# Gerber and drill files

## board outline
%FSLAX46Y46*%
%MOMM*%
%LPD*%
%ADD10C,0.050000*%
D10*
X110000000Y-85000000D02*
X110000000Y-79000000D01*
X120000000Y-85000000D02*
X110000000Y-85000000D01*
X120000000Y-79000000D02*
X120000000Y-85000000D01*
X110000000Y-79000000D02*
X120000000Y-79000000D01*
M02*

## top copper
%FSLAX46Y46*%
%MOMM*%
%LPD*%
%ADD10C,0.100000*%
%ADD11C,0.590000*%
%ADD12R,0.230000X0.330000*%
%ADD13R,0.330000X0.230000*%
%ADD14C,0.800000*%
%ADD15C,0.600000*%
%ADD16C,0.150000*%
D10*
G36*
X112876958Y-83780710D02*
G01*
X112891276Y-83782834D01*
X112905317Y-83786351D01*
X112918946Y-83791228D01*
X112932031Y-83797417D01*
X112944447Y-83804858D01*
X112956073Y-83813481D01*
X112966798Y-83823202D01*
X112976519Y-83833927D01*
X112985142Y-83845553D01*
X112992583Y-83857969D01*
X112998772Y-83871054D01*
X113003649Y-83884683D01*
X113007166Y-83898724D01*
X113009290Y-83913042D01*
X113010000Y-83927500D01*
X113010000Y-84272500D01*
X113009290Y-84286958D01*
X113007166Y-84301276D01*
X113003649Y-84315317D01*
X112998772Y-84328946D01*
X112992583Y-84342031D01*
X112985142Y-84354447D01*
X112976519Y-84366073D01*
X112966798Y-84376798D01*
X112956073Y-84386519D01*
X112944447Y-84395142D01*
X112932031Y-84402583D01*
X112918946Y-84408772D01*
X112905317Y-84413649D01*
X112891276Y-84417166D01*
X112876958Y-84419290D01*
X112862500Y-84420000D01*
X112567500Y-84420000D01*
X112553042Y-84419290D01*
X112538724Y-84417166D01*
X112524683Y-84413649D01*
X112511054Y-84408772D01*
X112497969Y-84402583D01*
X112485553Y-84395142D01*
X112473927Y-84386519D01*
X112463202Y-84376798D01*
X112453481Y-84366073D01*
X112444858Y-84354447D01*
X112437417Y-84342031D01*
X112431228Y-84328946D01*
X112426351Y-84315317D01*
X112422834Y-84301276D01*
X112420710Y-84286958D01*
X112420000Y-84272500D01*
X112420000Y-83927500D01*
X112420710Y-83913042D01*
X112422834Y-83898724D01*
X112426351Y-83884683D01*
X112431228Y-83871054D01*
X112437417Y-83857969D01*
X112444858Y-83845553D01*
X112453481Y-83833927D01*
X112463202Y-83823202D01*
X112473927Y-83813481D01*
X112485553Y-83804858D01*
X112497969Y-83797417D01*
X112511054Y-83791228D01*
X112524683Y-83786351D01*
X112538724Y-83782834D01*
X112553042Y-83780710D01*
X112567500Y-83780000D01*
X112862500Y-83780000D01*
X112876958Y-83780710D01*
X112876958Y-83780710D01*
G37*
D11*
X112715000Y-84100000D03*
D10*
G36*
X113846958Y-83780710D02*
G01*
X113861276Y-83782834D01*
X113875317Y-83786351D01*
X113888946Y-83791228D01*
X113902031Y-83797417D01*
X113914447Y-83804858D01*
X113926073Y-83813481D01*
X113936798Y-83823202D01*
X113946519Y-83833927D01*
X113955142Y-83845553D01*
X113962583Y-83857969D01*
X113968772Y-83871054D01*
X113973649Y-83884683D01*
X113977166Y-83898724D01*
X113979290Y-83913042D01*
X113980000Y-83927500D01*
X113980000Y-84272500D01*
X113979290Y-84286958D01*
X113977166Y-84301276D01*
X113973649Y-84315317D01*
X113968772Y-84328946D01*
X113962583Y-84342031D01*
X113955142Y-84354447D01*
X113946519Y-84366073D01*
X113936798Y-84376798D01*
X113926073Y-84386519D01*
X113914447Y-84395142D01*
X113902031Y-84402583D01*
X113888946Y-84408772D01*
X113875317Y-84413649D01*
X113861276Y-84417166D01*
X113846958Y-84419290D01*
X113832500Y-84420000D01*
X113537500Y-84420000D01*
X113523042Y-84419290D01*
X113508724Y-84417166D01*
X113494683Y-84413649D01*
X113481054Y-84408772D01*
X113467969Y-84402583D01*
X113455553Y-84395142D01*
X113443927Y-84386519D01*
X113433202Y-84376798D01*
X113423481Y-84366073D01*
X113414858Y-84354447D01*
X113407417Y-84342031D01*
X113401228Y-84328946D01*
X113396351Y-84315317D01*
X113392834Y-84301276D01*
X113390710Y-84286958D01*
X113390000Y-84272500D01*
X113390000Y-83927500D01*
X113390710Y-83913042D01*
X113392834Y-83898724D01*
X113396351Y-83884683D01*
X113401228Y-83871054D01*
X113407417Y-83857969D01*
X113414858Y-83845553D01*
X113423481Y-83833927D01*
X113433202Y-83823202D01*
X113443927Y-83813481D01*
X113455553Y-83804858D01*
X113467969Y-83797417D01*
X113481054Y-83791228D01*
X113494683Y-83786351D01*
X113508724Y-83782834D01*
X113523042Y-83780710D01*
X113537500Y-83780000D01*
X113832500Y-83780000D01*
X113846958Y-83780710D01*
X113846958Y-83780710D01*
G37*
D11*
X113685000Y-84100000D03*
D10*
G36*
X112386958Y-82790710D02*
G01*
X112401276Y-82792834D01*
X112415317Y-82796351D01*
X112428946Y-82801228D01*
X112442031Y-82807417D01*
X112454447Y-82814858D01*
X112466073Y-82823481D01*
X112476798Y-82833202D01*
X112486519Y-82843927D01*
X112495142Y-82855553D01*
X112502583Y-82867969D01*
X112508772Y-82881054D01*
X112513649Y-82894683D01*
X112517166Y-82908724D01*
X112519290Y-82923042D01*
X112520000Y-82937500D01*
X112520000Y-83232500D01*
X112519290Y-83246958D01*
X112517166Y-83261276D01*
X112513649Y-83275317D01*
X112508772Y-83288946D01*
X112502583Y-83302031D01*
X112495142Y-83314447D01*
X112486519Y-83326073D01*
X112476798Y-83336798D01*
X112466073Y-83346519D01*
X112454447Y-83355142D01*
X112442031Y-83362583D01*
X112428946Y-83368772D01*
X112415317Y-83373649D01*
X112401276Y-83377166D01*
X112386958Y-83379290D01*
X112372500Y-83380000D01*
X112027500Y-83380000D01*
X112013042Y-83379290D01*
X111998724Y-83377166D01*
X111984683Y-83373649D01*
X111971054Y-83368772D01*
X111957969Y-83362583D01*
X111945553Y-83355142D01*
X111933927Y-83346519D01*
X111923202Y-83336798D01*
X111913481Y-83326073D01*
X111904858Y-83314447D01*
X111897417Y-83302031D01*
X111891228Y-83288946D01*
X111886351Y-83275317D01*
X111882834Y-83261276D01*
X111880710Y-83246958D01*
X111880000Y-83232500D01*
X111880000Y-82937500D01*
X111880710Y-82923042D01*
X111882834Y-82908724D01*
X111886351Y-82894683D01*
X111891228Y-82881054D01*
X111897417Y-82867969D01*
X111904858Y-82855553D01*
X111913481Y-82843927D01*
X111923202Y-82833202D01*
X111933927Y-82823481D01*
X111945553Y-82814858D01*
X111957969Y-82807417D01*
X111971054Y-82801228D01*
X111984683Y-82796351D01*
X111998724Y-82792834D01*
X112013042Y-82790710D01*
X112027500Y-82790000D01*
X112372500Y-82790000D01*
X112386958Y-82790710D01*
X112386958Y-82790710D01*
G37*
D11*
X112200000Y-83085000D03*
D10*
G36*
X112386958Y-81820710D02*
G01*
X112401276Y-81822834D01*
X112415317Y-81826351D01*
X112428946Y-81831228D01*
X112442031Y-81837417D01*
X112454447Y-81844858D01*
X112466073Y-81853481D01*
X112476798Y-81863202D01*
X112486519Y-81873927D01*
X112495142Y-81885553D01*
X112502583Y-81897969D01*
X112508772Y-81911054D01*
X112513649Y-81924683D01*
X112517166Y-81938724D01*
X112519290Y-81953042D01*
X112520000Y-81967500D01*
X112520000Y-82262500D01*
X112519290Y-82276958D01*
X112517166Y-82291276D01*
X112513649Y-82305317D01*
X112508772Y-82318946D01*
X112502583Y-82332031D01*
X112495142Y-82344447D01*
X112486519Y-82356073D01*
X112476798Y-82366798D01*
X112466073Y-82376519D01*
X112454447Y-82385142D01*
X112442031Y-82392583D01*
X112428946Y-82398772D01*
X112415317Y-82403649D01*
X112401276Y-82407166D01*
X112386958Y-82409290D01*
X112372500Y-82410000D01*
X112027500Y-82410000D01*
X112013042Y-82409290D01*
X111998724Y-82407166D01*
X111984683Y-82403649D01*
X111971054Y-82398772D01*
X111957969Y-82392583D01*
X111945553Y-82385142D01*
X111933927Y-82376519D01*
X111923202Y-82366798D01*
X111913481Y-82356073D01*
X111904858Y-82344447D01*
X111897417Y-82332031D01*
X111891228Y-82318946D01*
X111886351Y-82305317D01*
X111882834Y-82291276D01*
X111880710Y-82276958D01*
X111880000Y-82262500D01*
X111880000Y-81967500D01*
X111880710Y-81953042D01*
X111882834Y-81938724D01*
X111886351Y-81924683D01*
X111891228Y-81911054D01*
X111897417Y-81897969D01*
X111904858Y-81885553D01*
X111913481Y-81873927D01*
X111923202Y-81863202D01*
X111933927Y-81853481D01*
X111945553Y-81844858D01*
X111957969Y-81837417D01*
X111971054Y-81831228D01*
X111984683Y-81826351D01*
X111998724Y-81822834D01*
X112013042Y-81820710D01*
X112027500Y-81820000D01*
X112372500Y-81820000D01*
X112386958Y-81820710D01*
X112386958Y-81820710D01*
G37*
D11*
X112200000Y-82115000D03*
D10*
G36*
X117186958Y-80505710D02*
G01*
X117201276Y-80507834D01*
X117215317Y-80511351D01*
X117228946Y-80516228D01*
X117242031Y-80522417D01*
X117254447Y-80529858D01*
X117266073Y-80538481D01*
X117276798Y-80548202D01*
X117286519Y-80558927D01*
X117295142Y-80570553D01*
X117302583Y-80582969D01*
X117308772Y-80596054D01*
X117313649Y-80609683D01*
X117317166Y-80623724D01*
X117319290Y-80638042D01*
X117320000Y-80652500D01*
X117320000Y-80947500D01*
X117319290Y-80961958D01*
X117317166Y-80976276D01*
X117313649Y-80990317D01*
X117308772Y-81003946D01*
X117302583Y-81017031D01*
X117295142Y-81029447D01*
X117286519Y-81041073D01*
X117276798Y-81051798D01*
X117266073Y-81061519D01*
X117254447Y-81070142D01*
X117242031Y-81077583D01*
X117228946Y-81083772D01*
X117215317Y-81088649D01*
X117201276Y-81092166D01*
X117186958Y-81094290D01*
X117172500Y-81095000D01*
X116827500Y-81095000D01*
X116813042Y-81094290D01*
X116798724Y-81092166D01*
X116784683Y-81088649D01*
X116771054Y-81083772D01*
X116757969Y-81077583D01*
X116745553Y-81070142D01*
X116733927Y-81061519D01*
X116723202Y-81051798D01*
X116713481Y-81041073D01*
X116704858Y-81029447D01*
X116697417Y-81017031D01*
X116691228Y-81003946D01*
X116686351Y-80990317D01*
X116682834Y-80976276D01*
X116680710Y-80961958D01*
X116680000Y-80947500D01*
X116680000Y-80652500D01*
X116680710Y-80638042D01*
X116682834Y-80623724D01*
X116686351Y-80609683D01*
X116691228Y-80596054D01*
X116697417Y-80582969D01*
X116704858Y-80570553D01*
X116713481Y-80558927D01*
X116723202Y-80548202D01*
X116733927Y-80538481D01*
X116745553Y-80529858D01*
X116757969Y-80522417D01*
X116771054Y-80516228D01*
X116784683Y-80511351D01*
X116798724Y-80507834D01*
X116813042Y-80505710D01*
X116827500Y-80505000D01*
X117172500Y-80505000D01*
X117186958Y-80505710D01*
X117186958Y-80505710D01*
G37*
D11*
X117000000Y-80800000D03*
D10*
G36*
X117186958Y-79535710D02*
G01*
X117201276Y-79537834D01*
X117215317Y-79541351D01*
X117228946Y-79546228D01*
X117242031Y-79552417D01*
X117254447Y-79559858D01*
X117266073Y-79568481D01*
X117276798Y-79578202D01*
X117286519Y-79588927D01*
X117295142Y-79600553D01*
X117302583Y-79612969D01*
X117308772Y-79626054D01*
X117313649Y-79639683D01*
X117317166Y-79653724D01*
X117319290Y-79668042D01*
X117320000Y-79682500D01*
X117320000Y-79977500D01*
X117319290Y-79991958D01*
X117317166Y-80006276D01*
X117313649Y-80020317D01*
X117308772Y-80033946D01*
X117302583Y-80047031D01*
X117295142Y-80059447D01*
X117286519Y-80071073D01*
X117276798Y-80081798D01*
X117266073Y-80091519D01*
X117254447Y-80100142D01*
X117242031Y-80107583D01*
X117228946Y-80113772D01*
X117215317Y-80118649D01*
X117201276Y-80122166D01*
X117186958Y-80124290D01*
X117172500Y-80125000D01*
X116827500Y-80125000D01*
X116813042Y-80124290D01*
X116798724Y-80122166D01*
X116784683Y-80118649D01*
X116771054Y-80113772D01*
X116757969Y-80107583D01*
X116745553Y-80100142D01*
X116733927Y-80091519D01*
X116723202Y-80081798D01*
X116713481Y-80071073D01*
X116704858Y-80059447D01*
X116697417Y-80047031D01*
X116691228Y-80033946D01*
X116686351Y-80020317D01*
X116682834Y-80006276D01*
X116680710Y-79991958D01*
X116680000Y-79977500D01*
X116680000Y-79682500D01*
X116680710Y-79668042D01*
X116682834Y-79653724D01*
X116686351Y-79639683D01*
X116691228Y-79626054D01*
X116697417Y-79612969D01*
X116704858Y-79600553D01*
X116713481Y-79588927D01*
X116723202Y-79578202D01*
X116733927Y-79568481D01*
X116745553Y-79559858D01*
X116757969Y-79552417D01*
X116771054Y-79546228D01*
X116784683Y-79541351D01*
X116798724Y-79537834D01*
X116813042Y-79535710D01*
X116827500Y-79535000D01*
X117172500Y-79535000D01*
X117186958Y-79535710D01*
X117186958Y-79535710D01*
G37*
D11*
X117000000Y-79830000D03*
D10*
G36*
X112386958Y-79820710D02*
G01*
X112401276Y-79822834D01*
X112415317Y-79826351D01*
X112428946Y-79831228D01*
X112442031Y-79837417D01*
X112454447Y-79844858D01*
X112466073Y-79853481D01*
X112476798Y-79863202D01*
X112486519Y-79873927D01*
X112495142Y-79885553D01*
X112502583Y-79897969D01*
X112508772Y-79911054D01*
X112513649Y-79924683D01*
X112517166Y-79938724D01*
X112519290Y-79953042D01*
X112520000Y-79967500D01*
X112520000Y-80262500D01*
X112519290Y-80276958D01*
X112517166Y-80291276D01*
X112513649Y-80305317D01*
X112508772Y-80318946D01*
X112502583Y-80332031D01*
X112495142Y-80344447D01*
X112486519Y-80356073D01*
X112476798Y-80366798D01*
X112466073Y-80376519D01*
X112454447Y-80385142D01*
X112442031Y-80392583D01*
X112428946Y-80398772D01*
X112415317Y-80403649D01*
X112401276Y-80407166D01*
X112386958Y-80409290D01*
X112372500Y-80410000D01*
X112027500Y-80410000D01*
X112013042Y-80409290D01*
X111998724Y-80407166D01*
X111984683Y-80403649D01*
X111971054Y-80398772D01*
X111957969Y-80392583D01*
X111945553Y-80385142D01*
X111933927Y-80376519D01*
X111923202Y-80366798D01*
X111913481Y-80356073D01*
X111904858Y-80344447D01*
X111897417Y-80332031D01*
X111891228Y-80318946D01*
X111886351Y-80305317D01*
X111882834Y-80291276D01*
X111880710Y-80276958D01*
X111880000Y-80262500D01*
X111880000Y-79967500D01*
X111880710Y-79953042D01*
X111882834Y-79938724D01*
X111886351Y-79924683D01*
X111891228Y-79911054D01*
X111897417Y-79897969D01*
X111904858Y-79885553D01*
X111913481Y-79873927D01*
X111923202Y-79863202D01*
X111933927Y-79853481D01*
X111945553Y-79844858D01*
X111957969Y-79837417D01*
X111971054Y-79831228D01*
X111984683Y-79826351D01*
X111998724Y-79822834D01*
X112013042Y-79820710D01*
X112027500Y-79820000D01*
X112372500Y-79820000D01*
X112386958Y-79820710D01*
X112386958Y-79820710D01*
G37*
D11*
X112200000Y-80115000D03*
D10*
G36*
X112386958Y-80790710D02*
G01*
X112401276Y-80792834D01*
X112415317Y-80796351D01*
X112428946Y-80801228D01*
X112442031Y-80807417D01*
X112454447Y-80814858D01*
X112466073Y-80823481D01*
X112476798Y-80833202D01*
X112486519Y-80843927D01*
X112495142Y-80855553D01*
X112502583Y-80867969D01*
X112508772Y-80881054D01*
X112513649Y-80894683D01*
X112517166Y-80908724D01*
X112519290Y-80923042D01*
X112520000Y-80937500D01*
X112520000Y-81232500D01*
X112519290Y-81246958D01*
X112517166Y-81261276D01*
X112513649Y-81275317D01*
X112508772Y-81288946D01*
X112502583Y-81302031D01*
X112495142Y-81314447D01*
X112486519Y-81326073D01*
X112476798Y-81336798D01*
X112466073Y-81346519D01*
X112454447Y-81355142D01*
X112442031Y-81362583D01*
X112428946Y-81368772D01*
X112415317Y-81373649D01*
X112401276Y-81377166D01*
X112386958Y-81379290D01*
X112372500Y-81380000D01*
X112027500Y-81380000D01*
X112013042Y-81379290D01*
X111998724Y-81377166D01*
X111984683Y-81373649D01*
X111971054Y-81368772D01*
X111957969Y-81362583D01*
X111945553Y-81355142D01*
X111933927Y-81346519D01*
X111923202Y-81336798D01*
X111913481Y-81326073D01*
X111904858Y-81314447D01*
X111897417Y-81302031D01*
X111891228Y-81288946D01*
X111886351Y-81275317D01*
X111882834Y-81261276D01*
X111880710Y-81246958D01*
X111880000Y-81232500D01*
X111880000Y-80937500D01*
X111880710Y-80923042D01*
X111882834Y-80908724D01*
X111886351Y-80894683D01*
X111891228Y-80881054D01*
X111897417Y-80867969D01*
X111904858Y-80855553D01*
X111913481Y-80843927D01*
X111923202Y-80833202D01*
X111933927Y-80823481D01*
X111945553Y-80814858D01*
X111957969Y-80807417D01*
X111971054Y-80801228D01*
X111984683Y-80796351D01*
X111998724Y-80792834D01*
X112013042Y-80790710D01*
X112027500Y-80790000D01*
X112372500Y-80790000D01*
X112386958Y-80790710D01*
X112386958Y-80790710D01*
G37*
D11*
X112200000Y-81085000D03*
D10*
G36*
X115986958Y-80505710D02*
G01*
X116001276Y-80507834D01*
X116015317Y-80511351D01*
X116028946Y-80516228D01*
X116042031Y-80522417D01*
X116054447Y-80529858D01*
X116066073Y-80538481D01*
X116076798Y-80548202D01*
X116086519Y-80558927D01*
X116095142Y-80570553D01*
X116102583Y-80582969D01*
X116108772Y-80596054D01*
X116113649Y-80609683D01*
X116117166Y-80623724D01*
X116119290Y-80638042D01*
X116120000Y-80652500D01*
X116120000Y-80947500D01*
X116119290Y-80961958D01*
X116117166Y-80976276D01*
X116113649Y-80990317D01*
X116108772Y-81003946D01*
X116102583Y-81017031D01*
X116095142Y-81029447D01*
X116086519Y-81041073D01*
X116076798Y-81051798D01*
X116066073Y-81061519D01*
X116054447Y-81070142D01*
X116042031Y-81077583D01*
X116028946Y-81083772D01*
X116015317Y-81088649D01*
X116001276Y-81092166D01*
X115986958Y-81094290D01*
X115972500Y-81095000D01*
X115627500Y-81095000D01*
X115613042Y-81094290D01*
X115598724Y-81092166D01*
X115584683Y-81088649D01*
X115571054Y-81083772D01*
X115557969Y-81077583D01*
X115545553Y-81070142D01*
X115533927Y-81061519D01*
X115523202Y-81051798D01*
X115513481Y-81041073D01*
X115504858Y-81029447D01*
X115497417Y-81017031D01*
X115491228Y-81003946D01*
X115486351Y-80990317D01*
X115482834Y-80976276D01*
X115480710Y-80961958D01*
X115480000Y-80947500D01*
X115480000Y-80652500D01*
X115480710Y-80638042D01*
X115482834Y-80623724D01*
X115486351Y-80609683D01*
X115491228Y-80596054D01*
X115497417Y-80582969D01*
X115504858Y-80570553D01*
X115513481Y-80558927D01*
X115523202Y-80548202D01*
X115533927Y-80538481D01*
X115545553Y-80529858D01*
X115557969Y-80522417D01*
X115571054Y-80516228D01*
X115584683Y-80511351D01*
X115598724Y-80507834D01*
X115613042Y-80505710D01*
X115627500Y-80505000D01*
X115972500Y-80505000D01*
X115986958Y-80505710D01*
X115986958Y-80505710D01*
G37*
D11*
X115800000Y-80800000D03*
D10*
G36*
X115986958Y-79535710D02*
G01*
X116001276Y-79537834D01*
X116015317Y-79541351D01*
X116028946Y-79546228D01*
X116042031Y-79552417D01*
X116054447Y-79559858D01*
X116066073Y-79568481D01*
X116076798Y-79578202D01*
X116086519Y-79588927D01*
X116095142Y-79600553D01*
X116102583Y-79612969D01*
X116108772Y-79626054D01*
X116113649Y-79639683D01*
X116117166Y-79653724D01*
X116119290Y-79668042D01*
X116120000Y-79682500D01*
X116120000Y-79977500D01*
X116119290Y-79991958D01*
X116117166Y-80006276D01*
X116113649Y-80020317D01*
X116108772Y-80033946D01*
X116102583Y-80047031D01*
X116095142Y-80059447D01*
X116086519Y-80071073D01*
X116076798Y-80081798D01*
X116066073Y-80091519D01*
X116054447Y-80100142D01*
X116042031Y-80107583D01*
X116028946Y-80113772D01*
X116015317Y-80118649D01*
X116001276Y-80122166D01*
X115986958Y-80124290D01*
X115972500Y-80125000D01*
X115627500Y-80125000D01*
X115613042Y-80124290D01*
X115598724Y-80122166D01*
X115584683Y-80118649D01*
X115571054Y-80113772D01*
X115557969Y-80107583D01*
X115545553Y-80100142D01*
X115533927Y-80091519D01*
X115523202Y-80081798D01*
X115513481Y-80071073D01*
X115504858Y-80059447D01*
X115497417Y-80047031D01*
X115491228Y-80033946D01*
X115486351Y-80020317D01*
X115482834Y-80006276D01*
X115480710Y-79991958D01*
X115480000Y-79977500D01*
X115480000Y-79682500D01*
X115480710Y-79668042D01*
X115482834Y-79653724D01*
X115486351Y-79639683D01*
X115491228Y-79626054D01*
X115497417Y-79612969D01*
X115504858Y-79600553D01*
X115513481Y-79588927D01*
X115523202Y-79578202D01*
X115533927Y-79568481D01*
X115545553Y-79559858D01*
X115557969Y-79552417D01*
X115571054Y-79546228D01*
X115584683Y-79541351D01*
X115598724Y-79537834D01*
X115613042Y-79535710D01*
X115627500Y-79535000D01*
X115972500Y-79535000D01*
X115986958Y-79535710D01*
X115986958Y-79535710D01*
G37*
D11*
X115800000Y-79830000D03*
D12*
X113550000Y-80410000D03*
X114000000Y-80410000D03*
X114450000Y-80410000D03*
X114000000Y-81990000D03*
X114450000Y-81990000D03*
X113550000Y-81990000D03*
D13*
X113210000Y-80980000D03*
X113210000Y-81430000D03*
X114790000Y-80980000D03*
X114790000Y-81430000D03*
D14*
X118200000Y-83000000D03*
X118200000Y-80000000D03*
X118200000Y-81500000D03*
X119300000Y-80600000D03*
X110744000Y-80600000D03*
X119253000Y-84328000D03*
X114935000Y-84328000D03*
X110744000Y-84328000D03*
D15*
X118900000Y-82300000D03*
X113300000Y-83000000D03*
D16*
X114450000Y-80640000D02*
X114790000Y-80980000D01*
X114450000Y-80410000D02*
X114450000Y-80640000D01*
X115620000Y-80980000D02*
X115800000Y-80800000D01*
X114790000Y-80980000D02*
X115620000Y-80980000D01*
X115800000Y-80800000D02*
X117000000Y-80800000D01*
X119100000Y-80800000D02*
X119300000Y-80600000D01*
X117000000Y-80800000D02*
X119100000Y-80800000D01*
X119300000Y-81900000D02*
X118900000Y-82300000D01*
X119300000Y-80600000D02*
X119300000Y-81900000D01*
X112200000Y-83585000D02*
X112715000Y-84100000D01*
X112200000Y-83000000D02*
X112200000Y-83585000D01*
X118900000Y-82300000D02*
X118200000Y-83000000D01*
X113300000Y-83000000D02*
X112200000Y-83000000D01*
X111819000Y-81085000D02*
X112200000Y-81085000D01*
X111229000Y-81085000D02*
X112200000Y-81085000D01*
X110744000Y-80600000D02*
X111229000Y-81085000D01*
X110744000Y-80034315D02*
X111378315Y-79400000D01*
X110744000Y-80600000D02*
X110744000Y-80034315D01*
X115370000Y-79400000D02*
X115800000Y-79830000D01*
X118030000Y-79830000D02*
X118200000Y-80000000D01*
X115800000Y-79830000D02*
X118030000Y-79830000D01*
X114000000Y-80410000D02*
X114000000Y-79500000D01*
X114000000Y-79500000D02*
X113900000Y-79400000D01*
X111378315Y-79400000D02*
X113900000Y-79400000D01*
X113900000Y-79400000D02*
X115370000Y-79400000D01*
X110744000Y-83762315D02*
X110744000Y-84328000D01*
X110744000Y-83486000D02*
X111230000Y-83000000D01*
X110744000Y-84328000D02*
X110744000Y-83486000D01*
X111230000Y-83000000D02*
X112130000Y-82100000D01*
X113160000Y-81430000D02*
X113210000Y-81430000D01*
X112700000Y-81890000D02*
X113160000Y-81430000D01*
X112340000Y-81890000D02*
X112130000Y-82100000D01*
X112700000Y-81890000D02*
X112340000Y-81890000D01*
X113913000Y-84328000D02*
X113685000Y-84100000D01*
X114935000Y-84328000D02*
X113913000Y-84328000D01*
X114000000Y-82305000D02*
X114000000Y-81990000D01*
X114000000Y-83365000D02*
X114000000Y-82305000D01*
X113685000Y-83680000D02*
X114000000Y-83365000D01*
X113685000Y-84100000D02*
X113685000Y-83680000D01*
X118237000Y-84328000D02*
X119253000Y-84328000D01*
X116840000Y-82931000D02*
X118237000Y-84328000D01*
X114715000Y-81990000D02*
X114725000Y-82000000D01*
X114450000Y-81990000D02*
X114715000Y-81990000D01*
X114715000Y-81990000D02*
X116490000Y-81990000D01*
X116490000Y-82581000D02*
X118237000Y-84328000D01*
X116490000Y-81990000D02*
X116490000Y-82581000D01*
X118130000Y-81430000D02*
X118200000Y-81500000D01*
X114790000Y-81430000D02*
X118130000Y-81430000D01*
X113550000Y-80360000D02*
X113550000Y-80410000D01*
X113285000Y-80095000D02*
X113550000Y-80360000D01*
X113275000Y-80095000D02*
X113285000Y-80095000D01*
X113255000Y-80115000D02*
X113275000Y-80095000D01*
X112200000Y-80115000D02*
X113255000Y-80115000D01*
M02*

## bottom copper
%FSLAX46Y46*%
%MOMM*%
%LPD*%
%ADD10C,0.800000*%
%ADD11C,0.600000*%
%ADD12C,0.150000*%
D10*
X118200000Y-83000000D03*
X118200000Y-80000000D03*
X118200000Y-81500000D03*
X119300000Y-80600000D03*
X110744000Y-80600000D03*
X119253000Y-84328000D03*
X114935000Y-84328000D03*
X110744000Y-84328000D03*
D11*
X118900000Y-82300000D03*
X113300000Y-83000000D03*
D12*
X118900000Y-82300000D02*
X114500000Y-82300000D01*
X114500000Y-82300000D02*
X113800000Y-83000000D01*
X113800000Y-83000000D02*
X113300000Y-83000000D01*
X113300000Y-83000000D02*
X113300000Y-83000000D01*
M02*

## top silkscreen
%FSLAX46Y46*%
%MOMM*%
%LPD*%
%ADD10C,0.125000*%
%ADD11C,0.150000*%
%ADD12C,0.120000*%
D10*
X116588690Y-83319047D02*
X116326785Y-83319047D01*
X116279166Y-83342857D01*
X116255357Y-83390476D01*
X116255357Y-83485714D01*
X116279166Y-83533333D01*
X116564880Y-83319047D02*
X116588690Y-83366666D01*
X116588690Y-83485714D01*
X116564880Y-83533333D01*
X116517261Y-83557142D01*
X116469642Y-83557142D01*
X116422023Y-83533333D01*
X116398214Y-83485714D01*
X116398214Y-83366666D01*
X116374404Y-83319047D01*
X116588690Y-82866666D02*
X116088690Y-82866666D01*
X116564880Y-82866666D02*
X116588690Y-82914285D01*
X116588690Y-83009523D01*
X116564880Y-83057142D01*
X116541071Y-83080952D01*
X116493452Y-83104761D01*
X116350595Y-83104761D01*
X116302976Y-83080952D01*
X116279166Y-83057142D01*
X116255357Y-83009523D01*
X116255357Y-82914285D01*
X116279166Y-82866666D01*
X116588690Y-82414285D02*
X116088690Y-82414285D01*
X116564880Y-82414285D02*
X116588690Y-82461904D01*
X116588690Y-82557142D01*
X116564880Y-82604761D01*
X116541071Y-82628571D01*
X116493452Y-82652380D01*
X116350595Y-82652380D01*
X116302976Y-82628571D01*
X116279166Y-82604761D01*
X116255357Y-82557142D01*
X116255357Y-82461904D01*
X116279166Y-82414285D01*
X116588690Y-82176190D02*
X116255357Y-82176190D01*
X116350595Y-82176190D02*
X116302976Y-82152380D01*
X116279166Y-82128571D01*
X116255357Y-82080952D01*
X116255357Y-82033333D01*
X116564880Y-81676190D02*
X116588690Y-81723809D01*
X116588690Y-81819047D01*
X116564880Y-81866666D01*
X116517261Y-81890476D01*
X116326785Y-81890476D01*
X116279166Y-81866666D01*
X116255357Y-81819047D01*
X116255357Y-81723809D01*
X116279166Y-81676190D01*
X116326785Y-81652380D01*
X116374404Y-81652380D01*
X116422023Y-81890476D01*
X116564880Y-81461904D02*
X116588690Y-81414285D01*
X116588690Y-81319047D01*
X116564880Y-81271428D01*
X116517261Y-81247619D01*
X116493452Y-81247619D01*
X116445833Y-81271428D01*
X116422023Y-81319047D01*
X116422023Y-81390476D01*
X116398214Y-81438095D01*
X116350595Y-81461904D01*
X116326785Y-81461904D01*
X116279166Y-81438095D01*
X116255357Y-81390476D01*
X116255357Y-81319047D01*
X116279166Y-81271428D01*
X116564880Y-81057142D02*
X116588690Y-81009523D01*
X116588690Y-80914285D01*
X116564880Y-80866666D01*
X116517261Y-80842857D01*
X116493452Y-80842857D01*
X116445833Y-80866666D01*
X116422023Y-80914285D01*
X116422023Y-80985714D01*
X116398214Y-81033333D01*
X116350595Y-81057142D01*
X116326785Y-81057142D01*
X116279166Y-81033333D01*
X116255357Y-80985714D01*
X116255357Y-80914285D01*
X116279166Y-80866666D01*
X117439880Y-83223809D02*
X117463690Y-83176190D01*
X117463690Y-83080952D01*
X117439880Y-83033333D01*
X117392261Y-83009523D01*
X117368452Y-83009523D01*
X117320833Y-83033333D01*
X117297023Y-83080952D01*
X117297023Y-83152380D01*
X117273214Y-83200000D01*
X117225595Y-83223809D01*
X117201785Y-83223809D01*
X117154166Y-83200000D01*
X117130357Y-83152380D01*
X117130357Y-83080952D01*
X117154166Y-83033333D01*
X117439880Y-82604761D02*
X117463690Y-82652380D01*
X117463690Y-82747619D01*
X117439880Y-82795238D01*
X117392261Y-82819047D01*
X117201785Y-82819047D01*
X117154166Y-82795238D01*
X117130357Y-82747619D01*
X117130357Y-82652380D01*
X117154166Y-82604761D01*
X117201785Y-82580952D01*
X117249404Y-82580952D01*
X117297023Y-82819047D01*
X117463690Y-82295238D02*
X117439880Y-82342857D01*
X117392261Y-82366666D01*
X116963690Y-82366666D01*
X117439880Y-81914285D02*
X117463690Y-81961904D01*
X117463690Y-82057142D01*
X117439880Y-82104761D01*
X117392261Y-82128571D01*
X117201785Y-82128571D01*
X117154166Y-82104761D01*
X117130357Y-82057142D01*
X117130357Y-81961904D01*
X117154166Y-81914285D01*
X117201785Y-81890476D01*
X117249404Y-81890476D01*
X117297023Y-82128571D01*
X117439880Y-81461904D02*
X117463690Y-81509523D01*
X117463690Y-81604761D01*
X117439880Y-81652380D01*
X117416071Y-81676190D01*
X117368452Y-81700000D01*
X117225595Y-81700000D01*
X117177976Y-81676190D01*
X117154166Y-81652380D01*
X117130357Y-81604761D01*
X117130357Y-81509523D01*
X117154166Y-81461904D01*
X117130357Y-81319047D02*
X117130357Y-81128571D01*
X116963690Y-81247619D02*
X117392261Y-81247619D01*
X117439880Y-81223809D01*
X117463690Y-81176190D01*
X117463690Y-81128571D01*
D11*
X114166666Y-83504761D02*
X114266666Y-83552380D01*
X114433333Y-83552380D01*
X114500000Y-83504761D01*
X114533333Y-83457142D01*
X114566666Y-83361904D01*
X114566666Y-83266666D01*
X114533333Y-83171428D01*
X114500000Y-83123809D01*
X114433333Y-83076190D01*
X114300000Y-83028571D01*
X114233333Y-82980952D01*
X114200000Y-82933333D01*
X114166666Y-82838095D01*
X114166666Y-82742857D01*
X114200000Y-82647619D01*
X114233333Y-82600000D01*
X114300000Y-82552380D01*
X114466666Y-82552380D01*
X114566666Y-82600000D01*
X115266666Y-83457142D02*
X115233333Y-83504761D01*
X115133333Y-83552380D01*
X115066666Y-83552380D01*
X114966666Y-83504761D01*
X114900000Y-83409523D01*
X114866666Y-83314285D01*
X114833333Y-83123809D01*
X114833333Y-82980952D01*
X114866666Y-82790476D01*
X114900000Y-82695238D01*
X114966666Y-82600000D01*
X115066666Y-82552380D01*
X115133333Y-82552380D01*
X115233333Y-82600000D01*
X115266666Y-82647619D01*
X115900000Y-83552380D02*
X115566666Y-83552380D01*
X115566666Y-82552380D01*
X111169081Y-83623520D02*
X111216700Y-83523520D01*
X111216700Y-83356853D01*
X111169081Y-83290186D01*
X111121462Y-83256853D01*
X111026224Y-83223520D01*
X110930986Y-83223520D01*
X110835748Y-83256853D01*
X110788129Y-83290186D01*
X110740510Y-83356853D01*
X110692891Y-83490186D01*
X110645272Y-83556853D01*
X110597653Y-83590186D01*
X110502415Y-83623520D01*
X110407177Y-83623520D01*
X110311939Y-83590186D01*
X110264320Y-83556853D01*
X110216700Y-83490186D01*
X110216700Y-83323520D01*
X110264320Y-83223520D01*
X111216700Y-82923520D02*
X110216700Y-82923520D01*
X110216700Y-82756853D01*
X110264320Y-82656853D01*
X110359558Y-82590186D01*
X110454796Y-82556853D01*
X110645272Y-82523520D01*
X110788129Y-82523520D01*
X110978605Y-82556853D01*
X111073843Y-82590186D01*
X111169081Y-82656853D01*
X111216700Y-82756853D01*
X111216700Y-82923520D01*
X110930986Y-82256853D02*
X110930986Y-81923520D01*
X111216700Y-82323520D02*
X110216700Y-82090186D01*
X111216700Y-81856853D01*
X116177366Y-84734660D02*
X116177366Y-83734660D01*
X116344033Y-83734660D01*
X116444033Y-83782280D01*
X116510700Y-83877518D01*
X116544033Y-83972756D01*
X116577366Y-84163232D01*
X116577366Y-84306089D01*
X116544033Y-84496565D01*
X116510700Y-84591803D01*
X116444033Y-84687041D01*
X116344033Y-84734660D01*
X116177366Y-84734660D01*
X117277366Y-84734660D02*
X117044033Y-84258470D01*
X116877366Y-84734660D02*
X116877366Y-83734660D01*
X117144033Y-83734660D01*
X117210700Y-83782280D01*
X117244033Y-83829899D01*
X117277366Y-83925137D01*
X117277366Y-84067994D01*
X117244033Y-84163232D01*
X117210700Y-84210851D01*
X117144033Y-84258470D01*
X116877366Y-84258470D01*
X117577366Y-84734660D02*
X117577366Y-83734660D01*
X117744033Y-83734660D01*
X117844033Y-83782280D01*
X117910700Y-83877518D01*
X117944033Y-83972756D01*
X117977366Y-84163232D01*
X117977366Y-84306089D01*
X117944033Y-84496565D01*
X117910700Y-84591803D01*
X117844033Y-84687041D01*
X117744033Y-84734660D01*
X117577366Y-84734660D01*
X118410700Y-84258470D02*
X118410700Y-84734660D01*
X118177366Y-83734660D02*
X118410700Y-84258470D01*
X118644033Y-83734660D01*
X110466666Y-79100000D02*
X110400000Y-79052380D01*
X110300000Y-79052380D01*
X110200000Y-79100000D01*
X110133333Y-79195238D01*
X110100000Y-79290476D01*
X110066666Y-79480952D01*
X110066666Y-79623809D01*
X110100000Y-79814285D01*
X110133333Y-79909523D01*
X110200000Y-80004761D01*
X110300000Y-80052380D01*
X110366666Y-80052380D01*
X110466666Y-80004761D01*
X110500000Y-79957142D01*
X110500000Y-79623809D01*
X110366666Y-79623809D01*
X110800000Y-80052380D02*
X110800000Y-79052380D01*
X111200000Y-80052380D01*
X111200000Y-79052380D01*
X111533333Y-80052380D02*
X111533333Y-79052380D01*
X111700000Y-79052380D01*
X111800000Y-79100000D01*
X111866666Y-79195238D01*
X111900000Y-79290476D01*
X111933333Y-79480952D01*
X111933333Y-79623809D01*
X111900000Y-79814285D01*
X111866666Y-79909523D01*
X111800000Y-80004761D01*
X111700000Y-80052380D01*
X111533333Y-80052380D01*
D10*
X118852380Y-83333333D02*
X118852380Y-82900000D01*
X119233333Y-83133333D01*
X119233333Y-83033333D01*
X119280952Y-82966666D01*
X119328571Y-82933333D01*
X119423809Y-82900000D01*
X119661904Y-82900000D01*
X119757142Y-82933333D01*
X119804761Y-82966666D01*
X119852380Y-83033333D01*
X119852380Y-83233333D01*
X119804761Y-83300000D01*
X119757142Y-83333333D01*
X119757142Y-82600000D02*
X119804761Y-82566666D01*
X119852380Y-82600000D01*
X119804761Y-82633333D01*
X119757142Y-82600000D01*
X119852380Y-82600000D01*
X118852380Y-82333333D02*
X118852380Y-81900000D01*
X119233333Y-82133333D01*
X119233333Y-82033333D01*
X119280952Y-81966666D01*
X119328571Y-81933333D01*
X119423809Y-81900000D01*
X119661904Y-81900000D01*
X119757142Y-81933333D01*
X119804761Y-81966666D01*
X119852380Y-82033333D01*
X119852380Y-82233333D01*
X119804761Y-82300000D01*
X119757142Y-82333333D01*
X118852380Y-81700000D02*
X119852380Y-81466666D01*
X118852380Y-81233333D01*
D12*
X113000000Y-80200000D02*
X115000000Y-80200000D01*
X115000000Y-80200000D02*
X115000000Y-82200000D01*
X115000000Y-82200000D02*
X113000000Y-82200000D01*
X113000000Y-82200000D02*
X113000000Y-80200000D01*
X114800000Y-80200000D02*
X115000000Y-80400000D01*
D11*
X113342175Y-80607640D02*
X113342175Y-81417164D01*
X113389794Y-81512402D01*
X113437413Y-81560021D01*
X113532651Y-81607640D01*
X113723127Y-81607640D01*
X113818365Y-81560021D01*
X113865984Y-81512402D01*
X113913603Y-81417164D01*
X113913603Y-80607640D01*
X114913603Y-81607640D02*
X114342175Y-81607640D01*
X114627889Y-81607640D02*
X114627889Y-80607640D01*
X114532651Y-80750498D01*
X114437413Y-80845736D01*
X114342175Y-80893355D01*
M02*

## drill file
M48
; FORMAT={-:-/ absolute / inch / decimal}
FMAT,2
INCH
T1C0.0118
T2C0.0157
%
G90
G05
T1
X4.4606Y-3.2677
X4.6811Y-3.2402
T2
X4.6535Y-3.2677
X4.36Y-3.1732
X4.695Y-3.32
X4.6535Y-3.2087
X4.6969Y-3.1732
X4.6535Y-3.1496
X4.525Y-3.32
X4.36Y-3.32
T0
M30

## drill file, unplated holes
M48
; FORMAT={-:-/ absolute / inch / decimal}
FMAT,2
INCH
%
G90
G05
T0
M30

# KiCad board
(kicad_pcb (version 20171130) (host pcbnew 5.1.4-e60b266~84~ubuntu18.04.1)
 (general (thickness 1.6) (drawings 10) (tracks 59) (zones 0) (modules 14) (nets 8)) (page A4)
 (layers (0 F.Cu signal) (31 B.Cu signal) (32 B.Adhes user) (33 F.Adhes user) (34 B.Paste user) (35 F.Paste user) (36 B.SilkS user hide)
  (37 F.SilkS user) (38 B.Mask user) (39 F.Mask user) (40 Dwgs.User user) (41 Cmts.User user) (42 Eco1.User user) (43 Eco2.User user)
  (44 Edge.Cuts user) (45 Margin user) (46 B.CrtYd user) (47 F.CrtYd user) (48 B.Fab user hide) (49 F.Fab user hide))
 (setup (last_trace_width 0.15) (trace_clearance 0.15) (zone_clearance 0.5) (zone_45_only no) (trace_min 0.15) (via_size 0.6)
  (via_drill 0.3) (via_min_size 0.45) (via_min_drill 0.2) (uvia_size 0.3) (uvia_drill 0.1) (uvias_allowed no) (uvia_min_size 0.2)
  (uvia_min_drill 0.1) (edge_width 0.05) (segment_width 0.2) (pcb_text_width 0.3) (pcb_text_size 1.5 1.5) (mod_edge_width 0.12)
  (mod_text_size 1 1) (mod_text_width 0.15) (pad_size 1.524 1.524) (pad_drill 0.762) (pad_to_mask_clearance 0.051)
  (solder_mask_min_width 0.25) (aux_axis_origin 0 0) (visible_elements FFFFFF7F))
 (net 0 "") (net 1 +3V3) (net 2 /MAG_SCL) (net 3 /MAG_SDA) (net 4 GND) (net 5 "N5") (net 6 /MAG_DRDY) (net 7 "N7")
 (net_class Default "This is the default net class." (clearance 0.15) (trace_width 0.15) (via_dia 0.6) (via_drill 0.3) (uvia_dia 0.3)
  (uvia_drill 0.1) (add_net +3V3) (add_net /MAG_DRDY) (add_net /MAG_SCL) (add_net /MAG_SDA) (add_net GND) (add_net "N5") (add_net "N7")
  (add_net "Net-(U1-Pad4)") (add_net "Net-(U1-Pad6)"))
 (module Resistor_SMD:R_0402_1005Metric (layer F.Cu) (at 113.2 84.1 180)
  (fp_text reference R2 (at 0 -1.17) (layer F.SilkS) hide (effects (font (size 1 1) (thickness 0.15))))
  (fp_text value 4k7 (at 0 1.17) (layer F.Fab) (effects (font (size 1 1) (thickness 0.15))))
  (pad 2 smd roundrect (at 0.485 0 180) (size 0.59 0.64) (layers F.Cu F.Paste F.Mask) (roundrect_rratio 0.25) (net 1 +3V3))
  (pad 1 smd roundrect (at -0.485 0 180) (size 0.59 0.64) (layers F.Cu F.Paste F.Mask) (roundrect_rratio 0.25) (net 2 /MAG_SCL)))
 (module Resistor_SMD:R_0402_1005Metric (layer F.Cu) (at 112.2 82.6 270)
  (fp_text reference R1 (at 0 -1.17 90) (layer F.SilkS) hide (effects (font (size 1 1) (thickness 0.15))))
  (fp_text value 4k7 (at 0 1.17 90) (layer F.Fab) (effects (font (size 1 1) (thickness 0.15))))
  (pad 2 smd roundrect (at 0.485 0 270) (size 0.59 0.64) (layers F.Cu F.Paste F.Mask) (roundrect_rratio 0.25) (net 1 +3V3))
  (pad 1 smd roundrect (at -0.485 0 270) (size 0.59 0.64) (layers F.Cu F.Paste F.Mask) (roundrect_rratio 0.25) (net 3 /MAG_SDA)))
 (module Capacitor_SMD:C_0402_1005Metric (layer F.Cu) (at 117 80.315 270)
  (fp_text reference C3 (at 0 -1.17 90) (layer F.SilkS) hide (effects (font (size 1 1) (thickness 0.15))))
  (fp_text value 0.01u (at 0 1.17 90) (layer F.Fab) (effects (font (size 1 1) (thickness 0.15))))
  (pad 2 smd roundrect (at 0.485 0 270) (size 0.59 0.64) (layers F.Cu F.Paste F.Mask) (roundrect_rratio 0.25) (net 1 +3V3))
  (pad 1 smd roundrect (at -0.485 0 270) (size 0.59 0.64) (layers F.Cu F.Paste F.Mask) (roundrect_rratio 0.25) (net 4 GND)))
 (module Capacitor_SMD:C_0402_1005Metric (layer F.Cu) (at 112.2 80.6 90)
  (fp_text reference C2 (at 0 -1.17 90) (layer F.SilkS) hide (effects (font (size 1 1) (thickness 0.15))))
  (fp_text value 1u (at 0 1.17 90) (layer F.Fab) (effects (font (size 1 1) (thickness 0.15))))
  (pad 2 smd roundrect (at 0.485 0 90) (size 0.59 0.64) (layers F.Cu F.Paste F.Mask) (roundrect_rratio 0.25) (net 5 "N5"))
  (pad 1 smd roundrect (at -0.485 0 90) (size 0.59 0.64) (layers F.Cu F.Paste F.Mask) (roundrect_rratio 0.25) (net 4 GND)))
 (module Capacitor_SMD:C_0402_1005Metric (layer F.Cu) (at 115.8 80.315 270)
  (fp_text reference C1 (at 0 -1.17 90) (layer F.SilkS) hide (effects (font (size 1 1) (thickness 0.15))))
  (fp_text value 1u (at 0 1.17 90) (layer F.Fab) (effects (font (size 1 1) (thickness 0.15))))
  (pad 2 smd roundrect (at 0.485 0 270) (size 0.59 0.64) (layers F.Cu F.Paste F.Mask) (roundrect_rratio 0.25) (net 1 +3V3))
  (pad 1 smd roundrect (at -0.485 0 270) (size 0.59 0.64) (layers F.Cu F.Paste F.Mask) (roundrect_rratio 0.25) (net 4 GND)))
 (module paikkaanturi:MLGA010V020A (layer F.Cu) (at 113 80.2)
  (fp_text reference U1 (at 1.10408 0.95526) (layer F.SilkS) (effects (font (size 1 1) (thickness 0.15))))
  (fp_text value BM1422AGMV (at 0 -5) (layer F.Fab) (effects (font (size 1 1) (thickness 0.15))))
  (fp_line (start 0 0) (end 2 0) (layer F.SilkS) (width 0.12)) (fp_line (start 2 0) (end 2 2) (layer F.SilkS) (width 0.12))
  (fp_line (start 2 2) (end 0 2) (layer F.SilkS) (width 0.12)) (fp_line (start 0 2) (end 0 0) (layer F.SilkS) (width 0.12))
  (fp_line (start 1.8 0) (end 2 0.2) (layer F.SilkS) (width 0.12))
  (pad 3 smd rect (at 0.55 0.21) (size 0.23 0.33) (layers F.Cu F.Paste F.Mask) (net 5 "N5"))
  (pad 2 smd rect (at 1 0.21) (size 0.23 0.33) (layers F.Cu F.Paste F.Mask) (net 4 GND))
  (pad 1 smd rect (at 1.45 0.21) (size 0.23 0.33) (layers F.Cu F.Paste F.Mask) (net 1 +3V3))
  (pad 7 smd rect (at 1 1.79) (size 0.23 0.33) (layers F.Cu F.Paste F.Mask) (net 2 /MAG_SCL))
  (pad 8 smd rect (at 1.45 1.79) (size 0.23 0.33) (layers F.Cu F.Paste F.Mask) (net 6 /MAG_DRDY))
  (pad 6 smd rect (at 0.55 1.79) (size 0.23 0.33) (layers F.Cu F.Paste F.Mask))
  (pad 4 smd rect (at 0.21 0.78 90) (size 0.23 0.33) (layers F.Cu F.Paste F.Mask))
  (pad 5 smd rect (at 0.21 1.23 90) (size 0.23 0.33) (layers F.Cu F.Paste F.Mask) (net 3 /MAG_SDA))
  (pad 10 smd rect (at 1.79 0.78 90) (size 0.23 0.33) (layers F.Cu F.Paste F.Mask) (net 1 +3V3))
  (pad 9 smd rect (at 1.79 1.23 90) (size 0.23 0.33) (layers F.Cu F.Paste F.Mask) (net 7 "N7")))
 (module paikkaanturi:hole (layer F.Cu) (at 118.2 83)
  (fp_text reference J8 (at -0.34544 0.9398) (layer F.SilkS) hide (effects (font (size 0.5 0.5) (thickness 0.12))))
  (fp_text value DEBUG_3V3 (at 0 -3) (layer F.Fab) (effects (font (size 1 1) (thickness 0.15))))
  (pad 1 thru_hole circle (at 0 0) (size 0.8 0.8) (drill 0.4) (layers *.Cu *.Mask) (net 1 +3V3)))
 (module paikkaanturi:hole (layer F.Cu) (at 118.2 80)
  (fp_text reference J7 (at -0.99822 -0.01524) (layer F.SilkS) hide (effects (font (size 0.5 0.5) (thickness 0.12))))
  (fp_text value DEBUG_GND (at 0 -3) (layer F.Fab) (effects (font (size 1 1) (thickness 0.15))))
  (pad 1 thru_hole circle (at 0 0) (size 0.8 0.8) (drill 0.4) (layers *.Cu *.Mask) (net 4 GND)))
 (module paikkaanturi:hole (layer F.Cu) (at 118.2 81.5)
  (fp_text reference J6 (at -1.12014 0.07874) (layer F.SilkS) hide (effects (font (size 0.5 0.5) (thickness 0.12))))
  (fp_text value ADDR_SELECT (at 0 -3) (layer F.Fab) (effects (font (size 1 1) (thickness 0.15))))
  (pad 1 thru_hole circle (at 0 0) (size 0.8 0.8) (drill 0.4) (layers *.Cu *.Mask) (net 7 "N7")))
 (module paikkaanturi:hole (layer F.Cu) (at 119.3 80.6)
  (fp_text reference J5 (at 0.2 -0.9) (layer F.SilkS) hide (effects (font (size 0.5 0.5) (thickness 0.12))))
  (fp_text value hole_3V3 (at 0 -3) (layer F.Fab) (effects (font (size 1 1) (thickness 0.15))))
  (pad 1 thru_hole circle (at 0 0) (size 0.8 0.8) (drill 0.4) (layers *.Cu *.Mask) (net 1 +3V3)))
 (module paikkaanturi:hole (layer F.Cu) (at 110.744 80.6)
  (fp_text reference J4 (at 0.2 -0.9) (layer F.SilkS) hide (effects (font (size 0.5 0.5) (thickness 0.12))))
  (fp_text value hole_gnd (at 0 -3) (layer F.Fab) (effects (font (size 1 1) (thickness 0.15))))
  (pad 1 thru_hole circle (at 0 0) (size 0.8 0.8) (drill 0.4) (layers *.Cu *.Mask) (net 4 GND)))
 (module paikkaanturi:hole (layer F.Cu) (at 119.253 84.328)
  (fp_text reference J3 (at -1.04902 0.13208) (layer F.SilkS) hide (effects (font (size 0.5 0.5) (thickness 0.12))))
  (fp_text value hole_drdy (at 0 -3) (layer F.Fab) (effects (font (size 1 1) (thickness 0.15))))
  (pad 1 thru_hole circle (at 0 0) (size 0.8 0.8) (drill 0.4) (layers *.Cu *.Mask) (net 6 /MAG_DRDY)))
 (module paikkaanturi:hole (layer F.Cu) (at 114.935 84.328)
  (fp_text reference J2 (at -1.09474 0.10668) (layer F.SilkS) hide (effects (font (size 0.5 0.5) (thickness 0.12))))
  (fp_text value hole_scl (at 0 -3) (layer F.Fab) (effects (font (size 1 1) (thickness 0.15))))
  (pad 1 thru_hole circle (at 0 0) (size 0.8 0.8) (drill 0.4) (layers *.Cu *.Mask) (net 2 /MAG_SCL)))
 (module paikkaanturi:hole (layer F.Cu) (at 110.744 84.328)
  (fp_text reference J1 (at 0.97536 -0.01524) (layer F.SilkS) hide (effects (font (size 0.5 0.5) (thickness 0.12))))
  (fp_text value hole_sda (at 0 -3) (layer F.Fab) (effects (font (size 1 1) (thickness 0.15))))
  (pad 1 thru_hole circle (at 0 0) (size 0.8 0.8) (drill 0.4) (layers *.Cu *.Mask) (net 3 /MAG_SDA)))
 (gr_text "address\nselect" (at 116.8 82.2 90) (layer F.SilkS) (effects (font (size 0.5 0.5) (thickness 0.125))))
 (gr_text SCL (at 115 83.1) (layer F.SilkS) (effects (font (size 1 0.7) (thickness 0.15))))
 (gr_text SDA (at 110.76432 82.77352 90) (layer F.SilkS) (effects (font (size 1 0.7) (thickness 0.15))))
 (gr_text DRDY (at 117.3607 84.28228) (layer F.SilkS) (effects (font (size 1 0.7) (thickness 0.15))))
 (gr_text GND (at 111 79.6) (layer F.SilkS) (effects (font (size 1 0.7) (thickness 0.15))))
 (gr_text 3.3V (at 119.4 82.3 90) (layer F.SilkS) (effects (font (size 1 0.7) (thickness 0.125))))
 (gr_line (start 110 85) (end 110 79) (layer Edge.Cuts) (width 0.05))
 (gr_line (start 120 85) (end 110 85) (layer Edge.Cuts) (width 0.05))
 (gr_line (start 120 79) (end 120 85) (layer Edge.Cuts) (width 0.05))
 (gr_line (start 110 79) (end 120 79) (layer Edge.Cuts) (width 0.05))
 (segment (start 114.45 80.64) (end 114.79 80.98) (width 0.15) (layer F.Cu) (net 1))
 (segment (start 114.45 80.41) (end 114.45 80.64) (width 0.15) (layer F.Cu) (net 1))
 (segment (start 115.62 80.98) (end 115.8 80.8) (width 0.15) (layer F.Cu) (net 1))
 (segment (start 114.79 80.98) (end 115.62 80.98) (width 0.15) (layer F.Cu) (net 1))
 (segment (start 115.8 80.8) (end 117 80.8) (width 0.15) (layer F.Cu) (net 1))
 (segment (start 119.1 80.8) (end 119.3 80.6) (width 0.15) (layer F.Cu) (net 1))
 (segment (start 117 80.8) (end 119.1 80.8) (width 0.15) (layer F.Cu) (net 1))
 (segment (start 119.3 81.9) (end 118.9 82.3) (width 0.15) (layer F.Cu) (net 1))
 (segment (start 119.3 80.6) (end 119.3 81.9) (width 0.15) (layer F.Cu) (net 1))
 (segment (start 112.2 83.585) (end 112.715 84.1) (width 0.15) (layer F.Cu) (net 1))
 (segment (start 112.2 83) (end 112.2 83.585) (width 0.15) (layer F.Cu) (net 1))
 (segment (start 118.9 82.3) (end 118.2 83) (width 0.15) (layer F.Cu) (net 1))
 (via (at 118.9 82.3) (size 0.6) (drill 0.3) (layers F.Cu B.Cu) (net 1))
 (segment (start 118.9 82.3) (end 114.5 82.3) (width 0.15) (layer B.Cu) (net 1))
 (segment (start 114.5 82.3) (end 113.8 83) (width 0.15) (layer B.Cu) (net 1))
 (segment (start 113.8 83) (end 113.3 83) (width 0.15) (layer B.Cu) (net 1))
 (segment (start 113.3 83) (end 113.3 83) (width 0.15) (layer B.Cu) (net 1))
 (via (at 113.3 83) (size 0.6) (drill 0.3) (layers F.Cu B.Cu) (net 1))
 (segment (start 113.3 83) (end 112.2 83) (width 0.15) (layer F.Cu) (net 1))
 (segment (start 111.819 81.085) (end 112.2 81.085) (width 0.15) (layer F.Cu) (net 4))
 (segment (start 111.229 81.085) (end 112.2 81.085) (width 0.15) (layer F.Cu) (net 4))
 (segment (start 110.744 80.6) (end 111.229 81.085) (width 0.15) (layer F.Cu) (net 4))
 (segment (start 110.744 80.034315) (end 111.378315 79.4) (width 0.15) (layer F.Cu) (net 4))
 (segment (start 110.744 80.6) (end 110.744 80.034315) (width 0.15) (layer F.Cu) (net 4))
 (segment (start 115.37 79.4) (end 115.8 79.83) (width 0.15) (layer F.Cu) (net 4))
 (segment (start 118.03 79.83) (end 118.2 80) (width 0.15) (layer F.Cu) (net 4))
 (segment (start 115.8 79.83) (end 118.03 79.83) (width 0.15) (layer F.Cu) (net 4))
 (segment (start 114 80.41) (end 114 79.5) (width 0.15) (layer F.Cu) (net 4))
 (segment (start 114 79.5) (end 113.9 79.4) (width 0.15) (layer F.Cu) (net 4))
 (segment (start 111.378315 79.4) (end 113.9 79.4) (width 0.15) (layer F.Cu) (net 4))
 (segment (start 113.9 79.4) (end 115.37 79.4) (width 0.15) (layer F.Cu) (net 4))
 (segment (start 110.744 83.762315) (end 110.744 84.328) (width 0.15) (layer F.Cu) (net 3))
 (segment (start 110.744 83.486) (end 111.23 83) (width 0.15) (layer F.Cu) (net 3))
 (segment (start 110.744 84.328) (end 110.744 83.486) (width 0.15) (layer F.Cu) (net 3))
 (segment (start 111.23 83) (end 112.13 82.1) (width 0.15) (layer F.Cu) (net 3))
 (segment (start 113.16 81.43) (end 113.21 81.43) (width 0.15) (layer F.Cu) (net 3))
 (segment (start 112.7 81.89) (end 113.16 81.43) (width 0.15) (layer F.Cu) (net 3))
 (segment (start 112.34 81.89) (end 112.13 82.1) (width 0.15) (layer F.Cu) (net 3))
 (segment (start 112.7 81.89) (end 112.34 81.89) (width 0.15) (layer F.Cu) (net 3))
 (segment (start 113.913 84.328) (end 113.685 84.1) (width 0.15) (layer F.Cu) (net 2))
 (segment (start 114.935 84.328) (end 113.913 84.328) (width 0.15) (layer F.Cu) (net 2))
 (segment (start 114 82.305) (end 114 81.99) (width 0.15) (layer F.Cu) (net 2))
 (segment (start 114 83.365) (end 114 82.305) (width 0.15) (layer F.Cu) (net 2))
 (segment (start 113.685 83.68) (end 114 83.365) (width 0.15) (layer F.Cu) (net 2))
 (segment (start 113.685 84.1) (end 113.685 83.68) (width 0.15) (layer F.Cu) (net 2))
 (segment (start 118.237 84.328) (end 119.253 84.328) (width 0.15) (layer F.Cu) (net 6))
 (segment (start 116.84 82.931) (end 118.237 84.328) (width 0.15) (layer F.Cu) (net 6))
 (segment (start 114.715 81.99) (end 114.725 82) (width 0.15) (layer F.Cu) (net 6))
 (segment (start 114.45 81.99) (end 114.715 81.99) (width 0.15) (layer F.Cu) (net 6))
 (segment (start 114.715 81.99) (end 116.49 81.99) (width 0.15) (layer F.Cu) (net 6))
 (segment (start 116.49 82.581) (end 118.237 84.328) (width 0.15) (layer F.Cu) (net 6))
 (segment (start 116.49 81.99) (end 116.49 82.581) (width 0.15) (layer F.Cu) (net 6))
 (segment (start 118.13 81.43) (end 118.2 81.5) (width 0.15) (layer F.Cu) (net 7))
 (segment (start 114.79 81.43) (end 118.13 81.43) (width 0.15) (layer F.Cu) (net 7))
 (segment (start 113.55 80.36) (end 113.55 80.41) (width 0.15) (layer F.Cu) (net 5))
 (segment (start 113.285 80.095) (end 113.55 80.36) (width 0.15) (layer F.Cu) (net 5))
 (segment (start 113.275 80.095) (end 113.285 80.095) (width 0.15) (layer F.Cu) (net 5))
 (segment (start 113.255 80.115) (end 113.275 80.095) (width 0.15) (layer F.Cu) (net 5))
 (segment (start 112.2 80.115) (end 113.255 80.115) (width 0.15) (layer F.Cu) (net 5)))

